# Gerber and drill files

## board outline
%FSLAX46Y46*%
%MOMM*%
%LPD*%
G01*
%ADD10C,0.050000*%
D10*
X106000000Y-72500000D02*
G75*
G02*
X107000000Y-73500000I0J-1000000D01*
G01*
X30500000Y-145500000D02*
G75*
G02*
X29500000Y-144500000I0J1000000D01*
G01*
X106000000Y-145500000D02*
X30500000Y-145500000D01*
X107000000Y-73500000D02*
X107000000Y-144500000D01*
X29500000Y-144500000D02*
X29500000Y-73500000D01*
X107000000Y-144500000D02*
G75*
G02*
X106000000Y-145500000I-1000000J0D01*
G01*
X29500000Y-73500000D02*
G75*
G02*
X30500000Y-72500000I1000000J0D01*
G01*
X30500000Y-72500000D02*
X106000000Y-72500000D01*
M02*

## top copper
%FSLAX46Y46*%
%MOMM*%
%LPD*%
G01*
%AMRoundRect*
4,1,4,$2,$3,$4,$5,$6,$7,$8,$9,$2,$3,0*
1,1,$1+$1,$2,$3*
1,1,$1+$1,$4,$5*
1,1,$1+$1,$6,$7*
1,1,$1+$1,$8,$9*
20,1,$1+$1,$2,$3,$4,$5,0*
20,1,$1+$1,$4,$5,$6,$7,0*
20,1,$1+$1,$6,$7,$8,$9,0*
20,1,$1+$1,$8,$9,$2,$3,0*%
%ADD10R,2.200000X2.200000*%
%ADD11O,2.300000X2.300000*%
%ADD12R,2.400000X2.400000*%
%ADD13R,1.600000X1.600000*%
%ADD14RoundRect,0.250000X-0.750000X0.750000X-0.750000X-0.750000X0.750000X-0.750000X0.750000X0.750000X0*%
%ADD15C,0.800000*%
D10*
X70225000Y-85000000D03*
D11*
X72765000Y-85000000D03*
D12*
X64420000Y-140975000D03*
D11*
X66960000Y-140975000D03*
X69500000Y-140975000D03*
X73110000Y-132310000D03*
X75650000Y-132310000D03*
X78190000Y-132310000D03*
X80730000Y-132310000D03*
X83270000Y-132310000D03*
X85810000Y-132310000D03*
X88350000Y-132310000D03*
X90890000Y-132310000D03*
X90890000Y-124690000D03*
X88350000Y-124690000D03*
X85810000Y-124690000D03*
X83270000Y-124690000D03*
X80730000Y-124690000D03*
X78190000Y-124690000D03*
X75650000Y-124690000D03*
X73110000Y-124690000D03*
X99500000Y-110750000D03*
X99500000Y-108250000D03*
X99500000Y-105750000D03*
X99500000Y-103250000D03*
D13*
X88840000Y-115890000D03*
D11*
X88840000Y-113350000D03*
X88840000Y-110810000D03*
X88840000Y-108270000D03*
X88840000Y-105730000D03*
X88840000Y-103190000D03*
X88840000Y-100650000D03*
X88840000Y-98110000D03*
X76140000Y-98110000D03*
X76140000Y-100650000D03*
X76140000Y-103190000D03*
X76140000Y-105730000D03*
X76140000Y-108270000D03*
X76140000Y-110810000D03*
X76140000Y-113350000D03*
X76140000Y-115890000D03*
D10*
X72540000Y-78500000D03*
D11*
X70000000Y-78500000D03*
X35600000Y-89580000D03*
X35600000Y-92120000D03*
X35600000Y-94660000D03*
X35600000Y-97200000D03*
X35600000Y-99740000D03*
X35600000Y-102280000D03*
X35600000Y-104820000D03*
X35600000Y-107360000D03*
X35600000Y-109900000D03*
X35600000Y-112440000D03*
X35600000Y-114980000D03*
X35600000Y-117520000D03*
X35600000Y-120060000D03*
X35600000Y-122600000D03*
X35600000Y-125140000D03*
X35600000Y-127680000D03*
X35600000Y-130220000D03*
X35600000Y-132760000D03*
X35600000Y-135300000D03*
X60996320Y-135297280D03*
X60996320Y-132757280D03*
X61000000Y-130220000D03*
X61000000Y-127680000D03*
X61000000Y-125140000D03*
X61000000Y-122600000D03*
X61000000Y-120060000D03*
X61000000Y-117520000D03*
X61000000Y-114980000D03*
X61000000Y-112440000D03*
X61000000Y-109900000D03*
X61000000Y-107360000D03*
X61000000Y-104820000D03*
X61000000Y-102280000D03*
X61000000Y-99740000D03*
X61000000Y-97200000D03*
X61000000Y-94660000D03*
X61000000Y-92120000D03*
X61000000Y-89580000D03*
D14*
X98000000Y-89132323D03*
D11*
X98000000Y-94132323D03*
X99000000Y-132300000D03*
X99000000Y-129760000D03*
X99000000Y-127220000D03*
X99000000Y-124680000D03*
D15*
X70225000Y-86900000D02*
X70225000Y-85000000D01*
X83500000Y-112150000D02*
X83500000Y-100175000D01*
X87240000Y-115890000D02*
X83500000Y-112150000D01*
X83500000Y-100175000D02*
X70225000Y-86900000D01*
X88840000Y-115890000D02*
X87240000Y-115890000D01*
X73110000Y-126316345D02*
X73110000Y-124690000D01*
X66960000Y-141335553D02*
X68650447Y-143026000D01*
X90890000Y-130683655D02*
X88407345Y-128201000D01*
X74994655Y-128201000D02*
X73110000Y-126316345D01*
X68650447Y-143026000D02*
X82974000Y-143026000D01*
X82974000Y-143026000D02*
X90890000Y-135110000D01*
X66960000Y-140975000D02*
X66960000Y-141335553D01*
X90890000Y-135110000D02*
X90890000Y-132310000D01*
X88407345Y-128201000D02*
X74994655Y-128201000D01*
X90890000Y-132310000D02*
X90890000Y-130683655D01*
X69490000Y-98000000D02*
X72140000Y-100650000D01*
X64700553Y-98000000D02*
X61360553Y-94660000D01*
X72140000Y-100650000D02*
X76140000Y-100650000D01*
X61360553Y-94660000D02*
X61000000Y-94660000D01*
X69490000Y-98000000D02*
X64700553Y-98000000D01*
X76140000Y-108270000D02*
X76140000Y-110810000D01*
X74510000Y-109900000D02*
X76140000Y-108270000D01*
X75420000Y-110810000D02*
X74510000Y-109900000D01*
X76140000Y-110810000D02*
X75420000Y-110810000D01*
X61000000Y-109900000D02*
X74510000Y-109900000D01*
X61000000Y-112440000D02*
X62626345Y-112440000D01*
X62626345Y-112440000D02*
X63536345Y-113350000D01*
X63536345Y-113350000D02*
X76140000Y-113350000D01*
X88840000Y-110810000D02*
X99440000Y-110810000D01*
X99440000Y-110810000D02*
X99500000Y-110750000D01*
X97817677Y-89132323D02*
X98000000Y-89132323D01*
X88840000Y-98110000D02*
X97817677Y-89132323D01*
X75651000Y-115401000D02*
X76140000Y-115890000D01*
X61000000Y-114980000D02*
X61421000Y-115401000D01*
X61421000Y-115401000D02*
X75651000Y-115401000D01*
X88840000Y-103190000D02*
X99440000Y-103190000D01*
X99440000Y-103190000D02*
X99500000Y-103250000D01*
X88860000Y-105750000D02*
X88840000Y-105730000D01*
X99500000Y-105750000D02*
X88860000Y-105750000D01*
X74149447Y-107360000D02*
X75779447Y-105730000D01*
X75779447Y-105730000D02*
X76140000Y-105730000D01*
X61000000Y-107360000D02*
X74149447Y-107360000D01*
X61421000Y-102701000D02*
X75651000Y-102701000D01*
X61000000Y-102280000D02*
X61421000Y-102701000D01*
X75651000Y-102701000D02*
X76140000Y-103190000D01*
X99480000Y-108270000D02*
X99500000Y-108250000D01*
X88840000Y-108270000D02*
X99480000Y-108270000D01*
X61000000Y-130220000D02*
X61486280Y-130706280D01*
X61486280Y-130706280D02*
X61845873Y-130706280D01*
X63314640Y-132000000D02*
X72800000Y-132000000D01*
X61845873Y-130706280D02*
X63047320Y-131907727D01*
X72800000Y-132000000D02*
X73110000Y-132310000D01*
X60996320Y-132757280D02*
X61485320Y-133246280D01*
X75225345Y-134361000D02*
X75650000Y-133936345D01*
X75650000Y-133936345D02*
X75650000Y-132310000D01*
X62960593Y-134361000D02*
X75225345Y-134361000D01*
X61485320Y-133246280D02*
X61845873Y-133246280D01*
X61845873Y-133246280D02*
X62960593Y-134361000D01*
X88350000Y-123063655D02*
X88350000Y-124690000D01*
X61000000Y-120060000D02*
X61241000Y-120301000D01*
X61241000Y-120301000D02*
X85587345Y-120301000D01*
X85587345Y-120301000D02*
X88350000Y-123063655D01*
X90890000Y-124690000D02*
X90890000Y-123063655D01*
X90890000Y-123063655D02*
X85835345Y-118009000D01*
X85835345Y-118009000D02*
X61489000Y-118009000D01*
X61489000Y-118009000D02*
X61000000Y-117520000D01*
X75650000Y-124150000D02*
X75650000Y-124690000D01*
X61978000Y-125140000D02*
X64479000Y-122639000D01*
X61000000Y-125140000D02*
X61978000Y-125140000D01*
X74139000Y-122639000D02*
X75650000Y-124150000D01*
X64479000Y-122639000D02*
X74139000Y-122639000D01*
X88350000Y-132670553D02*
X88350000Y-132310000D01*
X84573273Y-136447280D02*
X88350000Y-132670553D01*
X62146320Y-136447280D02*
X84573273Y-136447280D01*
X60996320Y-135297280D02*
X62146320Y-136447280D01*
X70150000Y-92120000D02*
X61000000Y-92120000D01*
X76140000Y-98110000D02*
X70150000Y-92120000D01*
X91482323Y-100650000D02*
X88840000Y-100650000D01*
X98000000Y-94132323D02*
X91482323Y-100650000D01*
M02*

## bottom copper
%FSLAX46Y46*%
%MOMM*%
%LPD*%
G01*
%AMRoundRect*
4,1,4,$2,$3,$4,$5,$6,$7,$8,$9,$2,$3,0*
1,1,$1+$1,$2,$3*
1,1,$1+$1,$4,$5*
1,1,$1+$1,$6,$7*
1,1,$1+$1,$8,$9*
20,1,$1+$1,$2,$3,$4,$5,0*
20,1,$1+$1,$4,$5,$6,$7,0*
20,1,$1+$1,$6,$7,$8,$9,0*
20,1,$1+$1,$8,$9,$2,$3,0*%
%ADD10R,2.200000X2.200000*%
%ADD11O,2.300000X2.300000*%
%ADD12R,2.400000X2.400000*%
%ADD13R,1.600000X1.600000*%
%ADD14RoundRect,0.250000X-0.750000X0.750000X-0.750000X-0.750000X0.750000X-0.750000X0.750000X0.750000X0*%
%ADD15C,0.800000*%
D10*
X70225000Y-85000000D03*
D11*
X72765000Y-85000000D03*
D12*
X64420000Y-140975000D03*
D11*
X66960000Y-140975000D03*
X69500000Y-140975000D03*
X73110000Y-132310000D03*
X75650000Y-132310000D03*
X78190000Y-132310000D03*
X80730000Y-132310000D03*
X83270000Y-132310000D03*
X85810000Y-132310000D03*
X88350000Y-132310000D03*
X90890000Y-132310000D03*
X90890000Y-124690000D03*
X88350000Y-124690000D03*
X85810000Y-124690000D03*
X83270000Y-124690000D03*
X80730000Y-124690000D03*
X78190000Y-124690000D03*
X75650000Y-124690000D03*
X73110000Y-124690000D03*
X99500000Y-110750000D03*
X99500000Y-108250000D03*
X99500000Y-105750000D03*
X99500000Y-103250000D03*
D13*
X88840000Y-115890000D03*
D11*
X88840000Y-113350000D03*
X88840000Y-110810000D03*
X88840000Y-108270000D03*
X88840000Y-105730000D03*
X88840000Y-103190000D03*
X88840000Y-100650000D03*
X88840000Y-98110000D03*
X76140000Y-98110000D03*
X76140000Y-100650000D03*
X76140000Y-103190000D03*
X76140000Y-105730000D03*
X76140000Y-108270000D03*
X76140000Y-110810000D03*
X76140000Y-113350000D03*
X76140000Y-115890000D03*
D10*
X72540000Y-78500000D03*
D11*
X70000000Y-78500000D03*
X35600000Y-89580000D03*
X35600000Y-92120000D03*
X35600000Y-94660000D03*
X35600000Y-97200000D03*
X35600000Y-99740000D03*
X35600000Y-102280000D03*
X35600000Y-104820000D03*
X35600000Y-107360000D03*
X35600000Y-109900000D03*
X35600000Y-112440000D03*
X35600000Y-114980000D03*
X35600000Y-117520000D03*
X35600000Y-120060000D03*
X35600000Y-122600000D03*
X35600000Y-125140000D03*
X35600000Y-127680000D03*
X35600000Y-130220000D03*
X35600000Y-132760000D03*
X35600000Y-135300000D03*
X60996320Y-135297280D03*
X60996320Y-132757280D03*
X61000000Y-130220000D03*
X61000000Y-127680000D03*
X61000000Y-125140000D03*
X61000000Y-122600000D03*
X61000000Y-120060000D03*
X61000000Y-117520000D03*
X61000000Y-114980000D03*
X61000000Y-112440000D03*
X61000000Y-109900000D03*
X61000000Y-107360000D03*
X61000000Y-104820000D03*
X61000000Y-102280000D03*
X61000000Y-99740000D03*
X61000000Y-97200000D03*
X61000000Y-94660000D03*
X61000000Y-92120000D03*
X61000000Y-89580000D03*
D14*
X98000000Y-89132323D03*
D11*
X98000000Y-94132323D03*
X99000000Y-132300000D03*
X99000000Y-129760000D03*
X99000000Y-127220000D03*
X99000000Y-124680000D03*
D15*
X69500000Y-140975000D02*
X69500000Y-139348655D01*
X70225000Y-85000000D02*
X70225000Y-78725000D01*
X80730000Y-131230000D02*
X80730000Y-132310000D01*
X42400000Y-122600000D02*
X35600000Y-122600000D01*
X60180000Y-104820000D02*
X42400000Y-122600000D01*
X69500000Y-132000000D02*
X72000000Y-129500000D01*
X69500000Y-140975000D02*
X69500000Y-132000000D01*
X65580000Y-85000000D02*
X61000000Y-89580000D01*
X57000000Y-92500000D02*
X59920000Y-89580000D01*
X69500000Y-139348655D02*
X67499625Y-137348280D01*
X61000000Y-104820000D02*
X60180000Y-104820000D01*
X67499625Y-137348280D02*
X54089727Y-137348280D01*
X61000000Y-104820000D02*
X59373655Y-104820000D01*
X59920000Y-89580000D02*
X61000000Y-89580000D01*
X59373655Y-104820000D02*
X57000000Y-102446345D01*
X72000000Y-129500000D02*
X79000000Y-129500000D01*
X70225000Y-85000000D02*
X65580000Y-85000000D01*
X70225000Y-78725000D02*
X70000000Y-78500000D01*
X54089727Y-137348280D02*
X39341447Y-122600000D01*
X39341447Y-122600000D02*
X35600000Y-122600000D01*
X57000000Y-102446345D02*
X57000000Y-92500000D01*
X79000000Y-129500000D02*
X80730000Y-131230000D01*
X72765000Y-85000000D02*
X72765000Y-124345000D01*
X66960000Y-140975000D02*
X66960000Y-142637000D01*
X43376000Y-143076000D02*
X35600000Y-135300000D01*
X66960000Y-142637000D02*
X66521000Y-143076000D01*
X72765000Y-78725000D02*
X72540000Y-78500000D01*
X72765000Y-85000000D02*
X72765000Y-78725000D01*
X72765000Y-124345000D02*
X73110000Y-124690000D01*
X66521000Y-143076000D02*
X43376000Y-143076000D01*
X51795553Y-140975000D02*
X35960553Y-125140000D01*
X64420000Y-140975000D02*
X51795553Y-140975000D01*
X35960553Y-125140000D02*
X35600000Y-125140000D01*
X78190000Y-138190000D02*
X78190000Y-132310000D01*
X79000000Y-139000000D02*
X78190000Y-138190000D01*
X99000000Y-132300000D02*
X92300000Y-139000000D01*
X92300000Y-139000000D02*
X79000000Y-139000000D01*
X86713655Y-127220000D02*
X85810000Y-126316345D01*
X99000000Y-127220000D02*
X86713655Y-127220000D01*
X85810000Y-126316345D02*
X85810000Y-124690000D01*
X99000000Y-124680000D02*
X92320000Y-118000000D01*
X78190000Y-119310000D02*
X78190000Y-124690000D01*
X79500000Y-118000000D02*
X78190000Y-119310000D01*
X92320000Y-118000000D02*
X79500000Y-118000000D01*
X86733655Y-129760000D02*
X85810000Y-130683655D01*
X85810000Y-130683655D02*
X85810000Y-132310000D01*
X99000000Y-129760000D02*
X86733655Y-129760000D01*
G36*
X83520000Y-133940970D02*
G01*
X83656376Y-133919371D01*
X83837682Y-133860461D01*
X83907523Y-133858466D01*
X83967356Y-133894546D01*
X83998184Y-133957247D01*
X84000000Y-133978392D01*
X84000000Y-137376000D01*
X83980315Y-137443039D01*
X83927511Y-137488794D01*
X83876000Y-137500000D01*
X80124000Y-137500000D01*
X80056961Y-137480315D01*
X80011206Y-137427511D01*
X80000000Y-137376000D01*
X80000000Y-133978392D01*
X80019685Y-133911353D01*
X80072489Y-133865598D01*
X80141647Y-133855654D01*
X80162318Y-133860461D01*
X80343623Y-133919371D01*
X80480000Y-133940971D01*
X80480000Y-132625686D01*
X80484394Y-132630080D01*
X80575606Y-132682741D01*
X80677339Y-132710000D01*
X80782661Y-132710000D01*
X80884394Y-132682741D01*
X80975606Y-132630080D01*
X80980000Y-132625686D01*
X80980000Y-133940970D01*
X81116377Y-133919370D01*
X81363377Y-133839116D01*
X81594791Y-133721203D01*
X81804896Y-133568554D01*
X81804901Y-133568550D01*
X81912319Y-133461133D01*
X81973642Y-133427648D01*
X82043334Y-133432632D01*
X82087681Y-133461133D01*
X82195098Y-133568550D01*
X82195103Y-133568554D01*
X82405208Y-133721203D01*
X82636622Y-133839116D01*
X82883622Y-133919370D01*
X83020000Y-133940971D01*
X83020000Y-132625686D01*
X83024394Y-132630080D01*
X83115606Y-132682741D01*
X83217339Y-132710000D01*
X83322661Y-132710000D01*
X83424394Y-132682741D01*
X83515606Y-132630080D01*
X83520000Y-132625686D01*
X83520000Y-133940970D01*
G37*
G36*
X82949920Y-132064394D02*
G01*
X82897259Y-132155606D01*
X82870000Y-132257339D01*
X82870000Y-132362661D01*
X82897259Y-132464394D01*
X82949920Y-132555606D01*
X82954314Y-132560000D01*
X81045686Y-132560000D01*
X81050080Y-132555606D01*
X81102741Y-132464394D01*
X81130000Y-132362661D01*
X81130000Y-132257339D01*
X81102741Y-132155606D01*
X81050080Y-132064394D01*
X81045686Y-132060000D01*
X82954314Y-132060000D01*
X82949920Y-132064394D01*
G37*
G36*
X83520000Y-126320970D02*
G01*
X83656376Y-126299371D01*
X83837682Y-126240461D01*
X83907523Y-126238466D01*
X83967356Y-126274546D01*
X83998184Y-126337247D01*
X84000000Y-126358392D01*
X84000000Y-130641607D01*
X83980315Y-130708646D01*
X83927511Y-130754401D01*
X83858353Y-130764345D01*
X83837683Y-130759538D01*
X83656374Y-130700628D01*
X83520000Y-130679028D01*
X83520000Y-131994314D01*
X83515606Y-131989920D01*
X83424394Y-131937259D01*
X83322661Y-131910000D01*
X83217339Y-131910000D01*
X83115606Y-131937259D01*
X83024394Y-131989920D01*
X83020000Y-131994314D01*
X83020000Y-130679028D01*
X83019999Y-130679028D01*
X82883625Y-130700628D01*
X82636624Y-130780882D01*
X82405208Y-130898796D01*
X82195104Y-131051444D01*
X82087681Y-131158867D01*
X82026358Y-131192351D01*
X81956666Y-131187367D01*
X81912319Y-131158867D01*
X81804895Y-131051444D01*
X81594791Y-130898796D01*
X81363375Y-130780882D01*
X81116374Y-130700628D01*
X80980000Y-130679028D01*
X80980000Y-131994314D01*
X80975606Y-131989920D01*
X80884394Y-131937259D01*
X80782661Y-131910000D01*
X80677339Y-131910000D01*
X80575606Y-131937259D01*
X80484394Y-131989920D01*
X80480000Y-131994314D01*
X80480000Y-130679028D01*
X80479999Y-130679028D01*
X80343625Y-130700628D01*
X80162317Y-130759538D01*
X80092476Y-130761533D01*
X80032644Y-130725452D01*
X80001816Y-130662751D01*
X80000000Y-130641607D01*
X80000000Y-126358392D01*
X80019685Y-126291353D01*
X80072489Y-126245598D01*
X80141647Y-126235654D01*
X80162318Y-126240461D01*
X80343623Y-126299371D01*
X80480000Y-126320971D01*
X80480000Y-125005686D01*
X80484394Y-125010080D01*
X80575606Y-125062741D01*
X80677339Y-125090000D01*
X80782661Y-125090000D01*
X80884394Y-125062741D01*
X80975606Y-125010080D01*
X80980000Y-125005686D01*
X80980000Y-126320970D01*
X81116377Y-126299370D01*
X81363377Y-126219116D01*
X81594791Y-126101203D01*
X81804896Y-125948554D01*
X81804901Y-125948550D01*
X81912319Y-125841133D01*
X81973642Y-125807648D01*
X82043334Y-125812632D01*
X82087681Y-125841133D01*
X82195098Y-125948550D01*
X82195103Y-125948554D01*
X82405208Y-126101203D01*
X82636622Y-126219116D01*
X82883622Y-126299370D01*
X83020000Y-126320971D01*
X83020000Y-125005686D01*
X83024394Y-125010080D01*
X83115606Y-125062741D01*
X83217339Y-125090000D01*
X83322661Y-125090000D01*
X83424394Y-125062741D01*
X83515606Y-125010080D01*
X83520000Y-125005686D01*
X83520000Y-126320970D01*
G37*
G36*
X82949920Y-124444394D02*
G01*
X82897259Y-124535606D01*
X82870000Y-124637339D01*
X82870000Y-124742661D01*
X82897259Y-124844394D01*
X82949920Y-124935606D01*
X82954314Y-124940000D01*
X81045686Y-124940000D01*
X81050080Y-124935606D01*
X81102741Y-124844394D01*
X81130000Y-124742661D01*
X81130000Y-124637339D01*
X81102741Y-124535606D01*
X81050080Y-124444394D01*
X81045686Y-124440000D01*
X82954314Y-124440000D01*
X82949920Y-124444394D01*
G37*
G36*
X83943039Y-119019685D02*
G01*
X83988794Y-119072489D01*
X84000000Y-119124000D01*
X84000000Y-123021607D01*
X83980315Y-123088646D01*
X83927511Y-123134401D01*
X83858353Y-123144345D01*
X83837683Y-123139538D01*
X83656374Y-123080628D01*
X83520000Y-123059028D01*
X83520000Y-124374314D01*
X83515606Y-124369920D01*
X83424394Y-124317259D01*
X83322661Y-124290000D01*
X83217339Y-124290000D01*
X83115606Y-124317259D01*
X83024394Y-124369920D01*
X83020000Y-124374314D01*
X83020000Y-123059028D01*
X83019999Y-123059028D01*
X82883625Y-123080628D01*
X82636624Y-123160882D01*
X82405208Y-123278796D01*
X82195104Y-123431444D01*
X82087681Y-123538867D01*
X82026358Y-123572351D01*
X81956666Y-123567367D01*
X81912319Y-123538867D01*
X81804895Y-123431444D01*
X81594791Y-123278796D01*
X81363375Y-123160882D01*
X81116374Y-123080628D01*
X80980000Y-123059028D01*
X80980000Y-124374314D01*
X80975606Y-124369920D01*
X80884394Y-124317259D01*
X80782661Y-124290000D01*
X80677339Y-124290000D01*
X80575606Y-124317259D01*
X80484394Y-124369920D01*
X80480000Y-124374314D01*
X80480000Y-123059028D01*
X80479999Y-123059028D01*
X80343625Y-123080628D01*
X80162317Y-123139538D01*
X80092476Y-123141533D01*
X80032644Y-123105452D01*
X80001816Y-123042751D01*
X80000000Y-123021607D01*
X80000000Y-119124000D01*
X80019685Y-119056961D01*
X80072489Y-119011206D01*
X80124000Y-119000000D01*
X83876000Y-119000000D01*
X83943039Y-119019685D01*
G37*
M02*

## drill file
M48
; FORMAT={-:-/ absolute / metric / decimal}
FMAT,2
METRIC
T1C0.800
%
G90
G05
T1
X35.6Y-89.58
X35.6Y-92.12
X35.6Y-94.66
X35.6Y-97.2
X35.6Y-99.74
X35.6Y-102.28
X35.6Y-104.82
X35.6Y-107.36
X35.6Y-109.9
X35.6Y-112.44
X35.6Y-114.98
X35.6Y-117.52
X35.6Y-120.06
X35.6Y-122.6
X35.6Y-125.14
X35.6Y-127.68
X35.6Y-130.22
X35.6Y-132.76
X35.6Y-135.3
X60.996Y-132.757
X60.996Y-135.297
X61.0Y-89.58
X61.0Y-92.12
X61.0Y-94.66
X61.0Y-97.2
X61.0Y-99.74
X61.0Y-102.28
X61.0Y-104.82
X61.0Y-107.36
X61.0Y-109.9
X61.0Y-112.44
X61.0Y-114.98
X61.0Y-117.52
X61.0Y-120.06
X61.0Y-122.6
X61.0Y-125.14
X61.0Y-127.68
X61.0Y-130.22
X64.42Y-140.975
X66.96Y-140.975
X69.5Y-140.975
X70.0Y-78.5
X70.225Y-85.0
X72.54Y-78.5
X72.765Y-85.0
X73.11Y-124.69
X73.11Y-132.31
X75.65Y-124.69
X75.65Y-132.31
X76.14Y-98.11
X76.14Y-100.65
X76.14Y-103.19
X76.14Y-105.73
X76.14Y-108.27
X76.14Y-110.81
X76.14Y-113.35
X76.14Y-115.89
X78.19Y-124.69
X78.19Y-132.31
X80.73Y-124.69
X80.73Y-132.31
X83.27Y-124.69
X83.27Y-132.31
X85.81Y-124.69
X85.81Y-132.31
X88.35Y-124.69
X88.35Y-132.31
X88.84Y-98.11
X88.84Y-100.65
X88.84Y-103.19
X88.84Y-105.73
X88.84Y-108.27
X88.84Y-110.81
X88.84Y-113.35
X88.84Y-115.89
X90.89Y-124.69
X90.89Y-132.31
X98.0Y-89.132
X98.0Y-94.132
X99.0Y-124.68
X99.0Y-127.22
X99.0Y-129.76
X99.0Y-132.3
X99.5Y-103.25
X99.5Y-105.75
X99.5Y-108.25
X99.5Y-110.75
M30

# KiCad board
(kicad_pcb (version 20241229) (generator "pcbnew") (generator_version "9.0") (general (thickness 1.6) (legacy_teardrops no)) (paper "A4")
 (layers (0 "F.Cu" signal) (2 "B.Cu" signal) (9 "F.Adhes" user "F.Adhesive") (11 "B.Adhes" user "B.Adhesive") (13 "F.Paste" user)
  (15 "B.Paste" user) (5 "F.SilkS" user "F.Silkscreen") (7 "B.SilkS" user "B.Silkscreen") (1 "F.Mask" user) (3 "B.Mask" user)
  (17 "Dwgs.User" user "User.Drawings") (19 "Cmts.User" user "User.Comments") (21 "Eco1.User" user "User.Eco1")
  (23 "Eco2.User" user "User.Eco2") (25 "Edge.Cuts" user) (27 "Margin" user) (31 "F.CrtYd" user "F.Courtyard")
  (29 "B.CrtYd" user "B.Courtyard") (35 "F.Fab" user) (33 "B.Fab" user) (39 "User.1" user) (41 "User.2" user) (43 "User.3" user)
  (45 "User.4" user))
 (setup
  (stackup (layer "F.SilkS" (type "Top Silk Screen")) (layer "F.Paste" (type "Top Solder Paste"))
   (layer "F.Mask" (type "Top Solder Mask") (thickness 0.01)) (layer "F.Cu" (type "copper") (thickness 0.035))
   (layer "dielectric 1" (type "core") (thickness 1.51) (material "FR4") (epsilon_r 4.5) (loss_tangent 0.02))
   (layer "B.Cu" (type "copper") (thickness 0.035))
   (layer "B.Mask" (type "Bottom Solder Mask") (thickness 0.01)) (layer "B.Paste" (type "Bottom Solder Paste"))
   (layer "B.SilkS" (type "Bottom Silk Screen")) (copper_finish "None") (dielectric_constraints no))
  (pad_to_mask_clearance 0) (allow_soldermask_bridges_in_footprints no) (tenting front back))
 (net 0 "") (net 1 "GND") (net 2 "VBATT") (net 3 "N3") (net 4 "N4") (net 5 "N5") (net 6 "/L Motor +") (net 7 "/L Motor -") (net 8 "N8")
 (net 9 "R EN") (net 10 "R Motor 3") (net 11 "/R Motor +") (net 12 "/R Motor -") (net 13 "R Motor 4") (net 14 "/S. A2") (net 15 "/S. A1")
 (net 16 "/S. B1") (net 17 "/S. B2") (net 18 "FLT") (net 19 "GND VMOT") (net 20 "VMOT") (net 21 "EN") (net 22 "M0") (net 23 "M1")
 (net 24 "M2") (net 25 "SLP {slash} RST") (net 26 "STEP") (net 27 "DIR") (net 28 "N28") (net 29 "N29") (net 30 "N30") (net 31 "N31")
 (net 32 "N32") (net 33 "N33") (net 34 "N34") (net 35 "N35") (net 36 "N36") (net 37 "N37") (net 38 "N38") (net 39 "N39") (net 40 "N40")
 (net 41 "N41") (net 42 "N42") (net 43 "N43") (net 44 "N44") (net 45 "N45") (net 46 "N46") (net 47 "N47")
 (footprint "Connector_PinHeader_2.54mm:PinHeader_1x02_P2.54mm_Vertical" (layer "F.Cu") (at 70.225 85 90)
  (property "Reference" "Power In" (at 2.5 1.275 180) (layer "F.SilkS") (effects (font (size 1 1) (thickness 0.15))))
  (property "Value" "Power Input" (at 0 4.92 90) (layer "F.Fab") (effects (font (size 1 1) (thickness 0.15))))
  (pad "1" thru_hole rect (at 0 0 90) (size 2.2 2.2) (drill 0.8) (layers "*.Cu" "*.Mask") (remove_unused_layers no) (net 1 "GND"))
  (pad "2" thru_hole oval (at 0 2.54 90) (size 2.3 2.3) (drill 0.8) (layers "*.Cu" "*.Mask") (remove_unused_layers no) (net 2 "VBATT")))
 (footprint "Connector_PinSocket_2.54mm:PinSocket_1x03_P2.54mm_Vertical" (layer "F.Cu") (at 64.42 140.975 90)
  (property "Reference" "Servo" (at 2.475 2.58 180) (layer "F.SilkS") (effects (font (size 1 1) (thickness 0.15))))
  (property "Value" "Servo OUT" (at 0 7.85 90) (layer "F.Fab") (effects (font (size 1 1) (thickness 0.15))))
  (pad "1" thru_hole rect (at 0 0 90) (size 2.4 2.4) (drill 0.8) (layers "*.Cu" "*.Mask") (remove_unused_layers no) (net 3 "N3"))
  (pad "2" thru_hole oval (at 0 2.54 90) (size 2.3 2.3) (drill 0.8) (layers "*.Cu" "*.Mask") (remove_unused_layers no) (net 2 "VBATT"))
  (pad "3" thru_hole oval (at 0 5.08 90) (size 2.3 2.3) (drill 0.8) (layers "*.Cu" "*.Mask") (remove_unused_layers no) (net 1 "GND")))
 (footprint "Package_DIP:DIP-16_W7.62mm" (layer "F.Cu") (at 73.11 132.31 90)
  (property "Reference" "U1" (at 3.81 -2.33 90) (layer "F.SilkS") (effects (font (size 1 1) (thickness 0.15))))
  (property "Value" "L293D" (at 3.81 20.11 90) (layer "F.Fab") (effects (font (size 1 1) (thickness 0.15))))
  (pad "1" thru_hole oval (at 0 0 90) (size 2.3 2.3) (drill 0.8) (layers "*.Cu" "*.Mask") (remove_unused_layers no) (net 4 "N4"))
  (pad "2" thru_hole oval (at 0 2.54 90) (size 2.3 2.3) (drill 0.8) (layers "*.Cu" "*.Mask") (remove_unused_layers no) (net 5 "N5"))
  (pad "3" thru_hole oval (at 0 5.08 90) (size 2.3 2.3) (drill 0.8) (layers "*.Cu" "*.Mask") (remove_unused_layers no) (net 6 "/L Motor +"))
  (pad "4" thru_hole oval (at 0 7.62 90) (size 2.3 2.3) (drill 0.8) (layers "*.Cu" "*.Mask") (remove_unused_layers no) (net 1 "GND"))
  (pad "5" thru_hole oval (at 0 10.16 90) (size 2.3 2.3) (drill 0.8) (layers "*.Cu" "*.Mask") (remove_unused_layers no) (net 1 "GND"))
  (pad "6" thru_hole oval (at 0 12.7 90) (size 2.3 2.3) (drill 0.8) (layers "*.Cu" "*.Mask") (remove_unused_layers no) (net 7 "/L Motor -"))
  (pad "7" thru_hole oval (at 0 15.24 90) (size 2.3 2.3) (drill 0.8) (layers "*.Cu" "*.Mask") (remove_unused_layers no) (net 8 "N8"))
  (pad "8" thru_hole oval (at 0 17.78 90) (size 2.3 2.3) (drill 0.8) (layers "*.Cu" "*.Mask") (remove_unused_layers no) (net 2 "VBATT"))
  (pad "9" thru_hole oval (at 7.62 17.78 90) (size 2.3 2.3) (drill 0.8) (layers "*.Cu" "*.Mask") (remove_unused_layers no) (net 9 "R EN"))
  (pad "10" thru_hole oval (at 7.62 15.24 90) (size 2.3 2.3) (drill 0.8) (layers "*.Cu" "*.Mask") (remove_unused_layers no)
   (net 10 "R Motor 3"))
  (pad "11" thru_hole oval (at 7.62 12.7 90) (size 2.3 2.3) (drill 0.8) (layers "*.Cu" "*.Mask") (remove_unused_layers no)
   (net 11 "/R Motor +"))
  (pad "12" thru_hole oval (at 7.62 10.16 90) (size 2.3 2.3) (drill 0.8) (layers "*.Cu" "*.Mask") (remove_unused_layers no) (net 1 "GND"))
  (pad "13" thru_hole oval (at 7.62 7.62 90) (size 2.3 2.3) (drill 0.8) (layers "*.Cu" "*.Mask") (remove_unused_layers no) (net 1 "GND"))
  (pad "14" thru_hole oval (at 7.62 5.08 90) (size 2.3 2.3) (drill 0.8) (layers "*.Cu" "*.Mask") (remove_unused_layers no)
   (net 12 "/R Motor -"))
  (pad "15" thru_hole oval (at 7.62 2.54 90) (size 2.3 2.3) (drill 0.8) (layers "*.Cu" "*.Mask") (remove_unused_layers no)
   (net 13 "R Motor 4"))
  (pad "16" thru_hole oval (at 7.62 0 90) (size 2.3 2.3) (drill 0.8) (layers "*.Cu" "*.Mask") (remove_unused_layers no) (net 2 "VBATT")))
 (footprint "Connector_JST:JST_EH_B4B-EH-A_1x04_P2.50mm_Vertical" (layer "F.Cu") (at 99.5 110.75 90)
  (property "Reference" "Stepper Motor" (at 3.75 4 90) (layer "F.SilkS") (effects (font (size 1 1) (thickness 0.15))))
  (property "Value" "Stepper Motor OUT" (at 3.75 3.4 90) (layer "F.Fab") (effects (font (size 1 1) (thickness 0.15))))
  (pad "1" thru_hole oval (at 0 0 90) (size 2.3 2.3) (drill 0.8) (layers "*.Cu" "*.Mask") (remove_unused_layers no) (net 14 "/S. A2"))
  (pad "2" thru_hole oval (at 2.5 0 90) (size 2.3 2.3) (drill 0.8) (layers "*.Cu" "*.Mask") (remove_unused_layers no) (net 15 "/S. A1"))
  (pad "3" thru_hole oval (at 5 0 90) (size 2.3 2.3) (drill 0.8) (layers "*.Cu" "*.Mask") (remove_unused_layers no) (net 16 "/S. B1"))
  (pad "4" thru_hole oval (at 7.5 0 90) (size 2.3 2.3) (drill 0.8) (layers "*.Cu" "*.Mask") (remove_unused_layers no) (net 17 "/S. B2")))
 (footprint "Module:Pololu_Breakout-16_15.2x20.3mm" (layer "F.Cu") (at 88.84 115.89 180)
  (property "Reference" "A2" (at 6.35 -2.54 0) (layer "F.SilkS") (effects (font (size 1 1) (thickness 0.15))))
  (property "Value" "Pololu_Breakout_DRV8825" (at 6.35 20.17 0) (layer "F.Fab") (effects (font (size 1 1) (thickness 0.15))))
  (pad "1" thru_hole rect (at 0 0 180) (size 1.6 1.6) (drill 0.8) (layers "*.Cu" "*.Mask") (remove_unused_layers no) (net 1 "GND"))
  (pad "2" thru_hole oval (at 0 2.54 180) (size 2.3 2.3) (drill 0.8) (layers "*.Cu" "*.Mask") (remove_unused_layers no) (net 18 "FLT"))
  (pad "3" thru_hole oval (at 0 5.08 180) (size 2.3 2.3) (drill 0.8) (layers "*.Cu" "*.Mask") (remove_unused_layers no) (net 14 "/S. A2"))
  (pad "4" thru_hole oval (at 0 7.62 180) (size 2.3 2.3) (drill 0.8) (layers "*.Cu" "*.Mask") (remove_unused_layers no) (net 15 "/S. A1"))
  (pad "5" thru_hole oval (at 0 10.16 180) (size 2.3 2.3) (drill 0.8) (layers "*.Cu" "*.Mask") (remove_unused_layers no) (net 16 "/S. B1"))
  (pad "6" thru_hole oval (at 0 12.7 180) (size 2.3 2.3) (drill 0.8) (layers "*.Cu" "*.Mask") (remove_unused_layers no) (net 17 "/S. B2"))
  (pad "7" thru_hole oval (at 0 15.24 180) (size 2.3 2.3) (drill 0.8) (layers "*.Cu" "*.Mask") (remove_unused_layers no) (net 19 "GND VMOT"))
  (pad "8" thru_hole oval (at 0 17.78 180) (size 2.3 2.3) (drill 0.8) (layers "*.Cu" "*.Mask") (remove_unused_layers no) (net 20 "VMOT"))
  (pad "9" thru_hole oval (at 12.7 17.78 180) (size 2.3 2.3) (drill 0.8) (layers "*.Cu" "*.Mask") (remove_unused_layers no) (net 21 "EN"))
  (pad "10" thru_hole oval (at 12.7 15.24 180) (size 2.3 2.3) (drill 0.8) (layers "*.Cu" "*.Mask") (remove_unused_layers no) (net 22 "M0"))
  (pad "11" thru_hole oval (at 12.7 12.7 180) (size 2.3 2.3) (drill 0.8) (layers "*.Cu" "*.Mask") (remove_unused_layers no) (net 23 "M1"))
  (pad "12" thru_hole oval (at 12.7 10.16 180) (size 2.3 2.3) (drill 0.8) (layers "*.Cu" "*.Mask") (remove_unused_layers no) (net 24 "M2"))
  (pad "13" thru_hole oval (at 12.7 7.62 180) (size 2.3 2.3) (drill 0.8) (layers "*.Cu" "*.Mask") (remove_unused_layers no)
   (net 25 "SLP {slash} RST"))
  (pad "14" thru_hole oval (at 12.7 5.08 180) (size 2.3 2.3) (drill 0.8) (layers "*.Cu" "*.Mask") (remove_unused_layers no)
   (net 25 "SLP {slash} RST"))
  (pad "15" thru_hole oval (at 12.7 2.54 180) (size 2.3 2.3) (drill 0.8) (layers "*.Cu" "*.Mask") (remove_unused_layers no) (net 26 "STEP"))
  (pad "16" thru_hole oval (at 12.7 0 180) (size 2.3 2.3) (drill 0.8) (layers "*.Cu" "*.Mask") (remove_unused_layers no) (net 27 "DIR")))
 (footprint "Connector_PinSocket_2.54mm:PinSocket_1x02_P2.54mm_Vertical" (layer "F.Cu") (at 72.54 78.5 -90)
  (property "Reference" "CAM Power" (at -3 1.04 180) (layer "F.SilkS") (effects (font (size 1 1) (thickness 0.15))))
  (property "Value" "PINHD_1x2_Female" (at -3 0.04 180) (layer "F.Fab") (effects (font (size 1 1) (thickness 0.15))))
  (pad "1" thru_hole rect (at 0 0 270) (size 2.2 2.2) (drill 0.8) (layers "*.Cu" "*.Mask") (remove_unused_layers no) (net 2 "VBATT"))
  (pad "2" thru_hole oval (at 0 2.54 270) (size 2.3 2.3) (drill 0.8) (layers "*.Cu" "*.Mask") (remove_unused_layers no) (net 1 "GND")))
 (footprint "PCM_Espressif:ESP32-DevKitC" (layer "F.Cu") (at 35.6 89.58)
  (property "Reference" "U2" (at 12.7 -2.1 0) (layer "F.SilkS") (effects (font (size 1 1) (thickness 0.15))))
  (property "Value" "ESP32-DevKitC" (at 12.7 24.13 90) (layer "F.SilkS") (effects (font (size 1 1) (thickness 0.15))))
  (pad "1" thru_hole oval (at 0 0) (size 2.3 2.3) (drill 0.8) (layers "*.Cu" "*.Mask") (remove_unused_layers no) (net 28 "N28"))
  (pad "2" thru_hole oval (at 0 2.54) (size 2.3 2.3) (drill 0.8) (layers "*.Cu" "*.Mask") (remove_unused_layers no) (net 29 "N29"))
  (pad "3" thru_hole oval (at 0 5.08) (size 2.3 2.3) (drill 0.8) (layers "*.Cu" "*.Mask") (remove_unused_layers no) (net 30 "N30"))
  (pad "4" thru_hole oval (at 0 7.62) (size 2.3 2.3) (drill 0.8) (layers "*.Cu" "*.Mask") (remove_unused_layers no) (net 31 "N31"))
  (pad "5" thru_hole oval (at 0 10.16) (size 2.3 2.3) (drill 0.8) (layers "*.Cu" "*.Mask") (remove_unused_layers no) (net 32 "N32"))
  (pad "6" thru_hole oval (at 0 12.7) (size 2.3 2.3) (drill 0.8) (layers "*.Cu" "*.Mask") (remove_unused_layers no) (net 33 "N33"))
  (pad "7" thru_hole oval (at 0 15.24) (size 2.3 2.3) (drill 0.8) (layers "*.Cu" "*.Mask") (remove_unused_layers no) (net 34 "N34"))
  (pad "8" thru_hole oval (at 0 17.78) (size 2.3 2.3) (drill 0.8) (layers "*.Cu" "*.Mask") (remove_unused_layers no) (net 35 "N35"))
  (pad "9" thru_hole oval (at 0 20.32) (size 2.3 2.3) (drill 0.8) (layers "*.Cu" "*.Mask") (remove_unused_layers no) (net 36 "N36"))
  (pad "10" thru_hole oval (at 0 22.86) (size 2.3 2.3) (drill 0.8) (layers "*.Cu" "*.Mask") (remove_unused_layers no) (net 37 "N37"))
  (pad "11" thru_hole oval (at 0 25.4) (size 2.3 2.3) (drill 0.8) (layers "*.Cu" "*.Mask") (remove_unused_layers no) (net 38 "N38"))
  (pad "12" thru_hole oval (at 0 27.94) (size 2.3 2.3) (drill 0.8) (layers "*.Cu" "*.Mask") (remove_unused_layers no) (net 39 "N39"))
  (pad "13" thru_hole oval (at 0 30.48) (size 2.3 2.3) (drill 0.8) (layers "*.Cu" "*.Mask") (remove_unused_layers no) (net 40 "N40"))
  (pad "14" thru_hole oval (at 0 33.02) (size 2.3 2.3) (drill 0.8) (layers "*.Cu" "*.Mask") (remove_unused_layers no) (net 1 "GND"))
  (pad "15" thru_hole oval (at 0 35.56) (size 2.3 2.3) (drill 0.8) (layers "*.Cu" "*.Mask") (remove_unused_layers no) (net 3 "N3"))
  (pad "16" thru_hole oval (at 0 38.1) (size 2.3 2.3) (drill 0.8) (layers "*.Cu" "*.Mask") (remove_unused_layers no) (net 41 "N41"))
  (pad "17" thru_hole oval (at 0 40.64) (size 2.3 2.3) (drill 0.8) (layers "*.Cu" "*.Mask") (remove_unused_layers no) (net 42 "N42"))
  (pad "18" thru_hole oval (at 0 43.18) (size 2.3 2.3) (drill 0.8) (layers "*.Cu" "*.Mask") (remove_unused_layers no) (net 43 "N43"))
  (pad "19" thru_hole oval (at 0 45.72) (size 2.3 2.3) (drill 0.8) (layers "*.Cu" "*.Mask") (remove_unused_layers no) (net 2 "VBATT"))
  (pad "20" thru_hole oval (at 25.39632 45.71728) (size 2.3 2.3) (drill 0.8) (layers "*.Cu" "*.Mask") (remove_unused_layers no) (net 8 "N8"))
  (pad "21" thru_hole oval (at 25.39632 43.17728) (size 2.3 2.3) (drill 0.8) (layers "*.Cu" "*.Mask") (remove_unused_layers no) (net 5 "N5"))
  (pad "22" thru_hole oval (at 25.4 40.64) (size 2.3 2.3) (drill 0.8) (layers "*.Cu" "*.Mask") (remove_unused_layers no) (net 4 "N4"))
  (pad "23" thru_hole oval (at 25.4 38.1) (size 2.3 2.3) (drill 0.8) (layers "*.Cu" "*.Mask") (remove_unused_layers no) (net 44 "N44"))
  (pad "24" thru_hole oval (at 25.4 35.56) (size 2.3 2.3) (drill 0.8) (layers "*.Cu" "*.Mask") (remove_unused_layers no)
   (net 13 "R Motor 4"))
  (pad "25" thru_hole oval (at 25.4 33.02) (size 2.3 2.3) (drill 0.8) (layers "*.Cu" "*.Mask") (remove_unused_layers no) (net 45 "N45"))
  (pad "26" thru_hole oval (at 25.4 30.48) (size 2.3 2.3) (drill 0.8) (layers "*.Cu" "*.Mask") (remove_unused_layers no)
   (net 10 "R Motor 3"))
  (pad "27" thru_hole oval (at 25.4 27.94) (size 2.3 2.3) (drill 0.8) (layers "*.Cu" "*.Mask") (remove_unused_layers no) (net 9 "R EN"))
  (pad "28" thru_hole oval (at 25.4 25.4) (size 2.3 2.3) (drill 0.8) (layers "*.Cu" "*.Mask") (remove_unused_layers no) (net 27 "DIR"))
  (pad "29" thru_hole oval (at 25.4 22.86) (size 2.3 2.3) (drill 0.8) (layers "*.Cu" "*.Mask") (remove_unused_layers no) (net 26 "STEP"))
  (pad "30" thru_hole oval (at 25.4 20.32) (size 2.3 2.3) (drill 0.8) (layers "*.Cu" "*.Mask") (remove_unused_layers no)
   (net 25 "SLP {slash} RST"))
  (pad "31" thru_hole oval (at 25.4 17.78) (size 2.3 2.3) (drill 0.8) (layers "*.Cu" "*.Mask") (remove_unused_layers no) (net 24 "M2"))
  (pad "32" thru_hole oval (at 25.4 15.24) (size 2.3 2.3) (drill 0.8) (layers "*.Cu" "*.Mask") (remove_unused_layers no) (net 1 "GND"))
  (pad "33" thru_hole oval (at 25.4 12.7) (size 2.3 2.3) (drill 0.8) (layers "*.Cu" "*.Mask") (remove_unused_layers no) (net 23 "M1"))
  (pad "34" thru_hole oval (at 25.4 10.16) (size 2.3 2.3) (drill 0.8) (layers "*.Cu" "*.Mask") (remove_unused_layers no) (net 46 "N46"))
  (pad "35" thru_hole oval (at 25.4 7.62) (size 2.3 2.3) (drill 0.8) (layers "*.Cu" "*.Mask") (remove_unused_layers no) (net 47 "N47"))
  (pad "36" thru_hole oval (at 25.4 5.08) (size 2.3 2.3) (drill 0.8) (layers "*.Cu" "*.Mask") (remove_unused_layers no) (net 22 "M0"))
  (pad "37" thru_hole oval (at 25.4 2.54) (size 2.3 2.3) (drill 0.8) (layers "*.Cu" "*.Mask") (remove_unused_layers no) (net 21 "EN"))
  (pad "38" thru_hole oval (at 25.4 0) (size 2.3 2.3) (drill 0.8) (layers "*.Cu" "*.Mask") (remove_unused_layers no) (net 1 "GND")))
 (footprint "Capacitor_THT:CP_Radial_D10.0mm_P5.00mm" (layer "F.Cu") (at 98 89.132323 -90)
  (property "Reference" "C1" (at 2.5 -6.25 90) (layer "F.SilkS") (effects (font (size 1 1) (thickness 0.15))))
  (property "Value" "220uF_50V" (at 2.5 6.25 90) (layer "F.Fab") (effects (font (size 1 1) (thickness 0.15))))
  (pad "1" thru_hole roundrect (at 0 0 270) (size 2 2) (drill 0.8) (layers "*.Cu" "*.Mask") (remove_unused_layers no)
   (roundrect_rratio 0.125) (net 20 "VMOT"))
  (pad "2" thru_hole oval (at 5 0 270) (size 2.3 2.3) (drill 0.8) (layers "*.Cu" "*.Mask") (remove_unused_layers no) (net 19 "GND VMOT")))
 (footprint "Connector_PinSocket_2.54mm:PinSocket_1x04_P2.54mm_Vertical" (layer "F.Cu") (at 99 132.3 180)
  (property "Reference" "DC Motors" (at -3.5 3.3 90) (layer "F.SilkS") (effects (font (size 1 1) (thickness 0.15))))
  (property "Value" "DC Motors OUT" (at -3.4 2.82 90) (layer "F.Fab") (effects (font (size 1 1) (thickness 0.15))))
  (pad "1" thru_hole oval (at 0 0 180) (size 2.3 2.3) (drill 0.8) (layers "*.Cu" "*.Mask") (remove_unused_layers no) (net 6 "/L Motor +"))
  (pad "2" thru_hole oval (at 0 2.54 180) (size 2.3 2.3) (drill 0.8) (layers "*.Cu" "*.Mask") (remove_unused_layers no) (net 7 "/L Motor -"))
  (pad "3" thru_hole oval (at 0 5.08 180) (size 2.3 2.3) (drill 0.8) (layers "*.Cu" "*.Mask") (remove_unused_layers no)
   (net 11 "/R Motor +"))
  (pad "4" thru_hole oval (at 0 7.62 180) (size 2.3 2.3) (drill 0.8) (layers "*.Cu" "*.Mask") (remove_unused_layers no)
   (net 12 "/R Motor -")))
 (gr_arc (start 106 72.5) (mid 106.707107 72.792893) (end 107 73.5) (stroke (width 0.05) (type default)) (layer "Edge.Cuts"))
 (gr_arc (start 30.5 145.5) (mid 29.792893 145.207107) (end 29.5 144.5) (stroke (width 0.05) (type default)) (layer "Edge.Cuts"))
 (gr_line (start 106 145.5) (end 30.5 145.5) (stroke (width 0.05) (type default)) (layer "Edge.Cuts"))
 (gr_line (start 107 73.5) (end 107 144.5) (stroke (width 0.05) (type default)) (layer "Edge.Cuts"))
 (gr_line (start 29.5 144.5) (end 29.5 73.5) (stroke (width 0.05) (type default)) (layer "Edge.Cuts"))
 (gr_arc (start 107 144.5) (mid 106.707107 145.207107) (end 106 145.5) (stroke (width 0.05) (type default)) (layer "Edge.Cuts"))
 (gr_arc (start 29.5 73.5) (mid 29.792893 72.792893) (end 30.5 72.5) (stroke (width 0.05) (type default)) (layer "Edge.Cuts"))
 (gr_line (start 30.5 72.5) (end 106 72.5) (stroke (width 0.05) (type default)) (layer "Edge.Cuts"))
 (segment (start 70.225 86.9) (end 70.225 85) (width 0.8) (layer "F.Cu") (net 1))
 (segment (start 83.5 112.15) (end 83.5 100.175) (width 0.8) (layer "F.Cu") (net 1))
 (segment (start 87.24 115.89) (end 83.5 112.15) (width 0.8) (layer "F.Cu") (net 1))
 (segment (start 83.5 100.175) (end 70.225 86.9) (width 0.8) (layer "F.Cu") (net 1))
 (segment (start 88.84 115.89) (end 87.24 115.89) (width 0.8) (layer "F.Cu") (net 1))
 (segment (start 69.5 140.975) (end 69.5 139.348655) (width 0.8) (layer "B.Cu") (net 1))
 (segment (start 70.225 85) (end 70.225 78.725) (width 0.8) (layer "B.Cu") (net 1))
 (segment (start 80.73 131.23) (end 80.73 132.31) (width 0.8) (layer "B.Cu") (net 1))
 (segment (start 42.4 122.6) (end 35.6 122.6) (width 0.8) (layer "B.Cu") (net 1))
 (segment (start 60.18 104.82) (end 42.4 122.6) (width 0.8) (layer "B.Cu") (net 1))
 (segment (start 69.5 132) (end 72 129.5) (width 0.8) (layer "B.Cu") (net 1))
 (segment (start 69.5 140.975) (end 69.5 132) (width 0.8) (layer "B.Cu") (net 1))
 (segment (start 65.58 85) (end 61 89.58) (width 0.8) (layer "B.Cu") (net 1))
 (segment (start 57 92.5) (end 59.92 89.58) (width 0.8) (layer "B.Cu") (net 1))
 (segment (start 69.5 139.348655) (end 67.499625 137.34828) (width 0.8) (layer "B.Cu") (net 1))
 (segment (start 61 104.82) (end 60.18 104.82) (width 0.8) (layer "B.Cu") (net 1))
 (segment (start 67.499625 137.34828) (end 54.089727 137.34828) (width 0.8) (layer "B.Cu") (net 1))
 (segment (start 61 104.82) (end 59.373655 104.82) (width 0.8) (layer "B.Cu") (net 1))
 (segment (start 59.92 89.58) (end 61 89.58) (width 0.8) (layer "B.Cu") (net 1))
 (segment (start 59.373655 104.82) (end 57 102.446345) (width 0.8) (layer "B.Cu") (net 1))
 (segment (start 72 129.5) (end 79 129.5) (width 0.8) (layer "B.Cu") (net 1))
 (segment (start 70.225 85) (end 65.58 85) (width 0.8) (layer "B.Cu") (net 1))
 (segment (start 70.225 78.725) (end 70 78.5) (width 0.8) (layer "B.Cu") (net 1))
 (segment (start 54.089727 137.34828) (end 39.341447 122.6) (width 0.8) (layer "B.Cu") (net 1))
 (segment (start 39.341447 122.6) (end 35.6 122.6) (width 0.8) (layer "B.Cu") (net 1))
 (segment (start 57 102.446345) (end 57 92.5) (width 0.8) (layer "B.Cu") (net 1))
 (segment (start 79 129.5) (end 80.73 131.23) (width 0.8) (layer "B.Cu") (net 1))
 (segment (start 73.11 126.316345) (end 73.11 124.69) (width 0.8) (layer "F.Cu") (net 2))
 (segment (start 66.96 141.335553) (end 68.650447 143.026) (width 0.8) (layer "F.Cu") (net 2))
 (segment (start 90.89 130.683655) (end 88.407345 128.201) (width 0.8) (layer "F.Cu") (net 2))
 (segment (start 74.994655 128.201) (end 73.11 126.316345) (width 0.8) (layer "F.Cu") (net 2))
 (segment (start 68.650447 143.026) (end 82.974 143.026) (width 0.8) (layer "F.Cu") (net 2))
 (segment (start 82.974 143.026) (end 90.89 135.11) (width 0.8) (layer "F.Cu") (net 2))
 (segment (start 66.96 140.975) (end 66.96 141.335553) (width 0.8) (layer "F.Cu") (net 2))
 (segment (start 90.89 135.11) (end 90.89 132.31) (width 0.8) (layer "F.Cu") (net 2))
 (segment (start 88.407345 128.201) (end 74.994655 128.201) (width 0.8) (layer "F.Cu") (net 2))
 (segment (start 90.89 132.31) (end 90.89 130.683655) (width 0.8) (layer "F.Cu") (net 2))
 (segment (start 72.765 85) (end 72.765 124.345) (width 0.8) (layer "B.Cu") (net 2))
 (segment (start 66.96 140.975) (end 66.96 142.637) (width 0.8) (layer "B.Cu") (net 2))
 (segment (start 43.376 143.076) (end 35.6 135.3) (width 0.8) (layer "B.Cu") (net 2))
 (segment (start 66.96 142.637) (end 66.521 143.076) (width 0.8) (layer "B.Cu") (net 2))
 (segment (start 72.765 78.725) (end 72.54 78.5) (width 0.8) (layer "B.Cu") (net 2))
 (segment (start 72.765 85) (end 72.765 78.725) (width 0.8) (layer "B.Cu") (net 2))
 (segment (start 72.765 124.345) (end 73.11 124.69) (width 0.8) (layer "B.Cu") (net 2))
 (segment (start 66.521 143.076) (end 43.376 143.076) (width 0.8) (layer "B.Cu") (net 2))
 (segment (start 69.49 98) (end 72.14 100.65) (width 0.8) (layer "F.Cu") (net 22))
 (segment (start 64.700553 98) (end 61.360553 94.66) (width 0.8) (layer "F.Cu") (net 22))
 (segment (start 72.14 100.65) (end 76.14 100.65) (width 0.8) (layer "F.Cu") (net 22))
 (segment (start 61.360553 94.66) (end 61 94.66) (width 0.8) (layer "F.Cu") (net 22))
 (segment (start 69.49 98) (end 64.700553 98) (width 0.8) (layer "F.Cu") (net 22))
 (segment (start 76.14 108.27) (end 76.14 110.81) (width 0.8) (layer "F.Cu") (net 25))
 (segment (start 74.51 109.9) (end 76.14 108.27) (width 0.8) (layer "F.Cu") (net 25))
 (segment (start 75.42 110.81) (end 74.51 109.9) (width 0.8) (layer "F.Cu") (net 25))
 (segment (start 76.14 110.81) (end 75.42 110.81) (width 0.8) (layer "F.Cu") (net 25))
 (segment (start 61 109.9) (end 74.51 109.9) (width 0.8) (layer "F.Cu") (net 25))
 (segment (start 61 112.44) (end 62.626345 112.44) (width 0.8) (layer "F.Cu") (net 26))
 (segment (start 62.626345 112.44) (end 63.536345 113.35) (width 0.8) (layer "F.Cu") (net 26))
 (segment (start 63.536345 113.35) (end 76.14 113.35) (width 0.8) (layer "F.Cu") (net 26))
 (segment (start 88.84 110.81) (end 99.44 110.81) (width 0.8) (layer "F.Cu") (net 14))
 (segment (start 99.44 110.81) (end 99.5 110.75) (width 0.8) (layer "F.Cu") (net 14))
 (segment (start 97.817677 89.132323) (end 98 89.132323) (width 0.8) (layer "F.Cu") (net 20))
 (segment (start 88.84 98.11) (end 97.817677 89.132323) (width 0.8) (layer "F.Cu") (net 20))
 (segment (start 75.651 115.401) (end 76.14 115.89) (width 0.8) (layer "F.Cu") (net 27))
 (segment (start 61 114.98) (end 61.421 115.401) (width 0.8) (layer "F.Cu") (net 27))
 (segment (start 61.421 115.401) (end 75.651 115.401) (width 0.8) (layer "F.Cu") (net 27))
 (segment (start 88.84 103.19) (end 99.44 103.19) (width 0.8) (layer "F.Cu") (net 17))
 (segment (start 99.44 103.19) (end 99.5 103.25) (width 0.8) (layer "F.Cu") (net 17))
 (segment (start 88.86 105.75) (end 88.84 105.73) (width 0.8) (layer "F.Cu") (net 16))
 (segment (start 99.5 105.75) (end 88.86 105.75) (width 0.8) (layer "F.Cu") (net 16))
 (segment (start 74.149447 107.36) (end 75.779447 105.73) (width 0.8) (layer "F.Cu") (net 24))
 (segment (start 75.779447 105.73) (end 76.14 105.73) (width 0.8) (layer "F.Cu") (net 24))
 (segment (start 61 107.36) (end 74.149447 107.36) (width 0.8) (layer "F.Cu") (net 24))
 (segment (start 61.421 102.701) (end 75.651 102.701) (width 0.8) (layer "F.Cu") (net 23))
 (segment (start 61 102.28) (end 61.421 102.701) (width 0.8) (layer "F.Cu") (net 23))
 (segment (start 75.651 102.701) (end 76.14 103.19) (width 0.8) (layer "F.Cu") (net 23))
 (segment (start 51.795553 140.975) (end 35.960553 125.14) (width 0.8) (layer "B.Cu") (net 3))
 (segment (start 64.42 140.975) (end 51.795553 140.975) (width 0.8) (layer "B.Cu") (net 3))
 (segment (start 35.960553 125.14) (end 35.6 125.14) (width 0.8) (layer "B.Cu") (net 3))
 (segment (start 99.48 108.27) (end 99.5 108.25) (width 0.8) (layer "F.Cu") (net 15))
 (segment (start 88.84 108.27) (end 99.48 108.27) (width 0.8) (layer "F.Cu") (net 15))
 (segment (start 78.19 138.19) (end 78.19 132.31) (width 0.8) (layer "B.Cu") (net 6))
 (segment (start 79 139) (end 78.19 138.19) (width 0.8) (layer "B.Cu") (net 6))
 (segment (start 99 132.3) (end 92.3 139) (width 0.8) (layer "B.Cu") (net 6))
 (segment (start 92.3 139) (end 79 139) (width 0.8) (layer "B.Cu") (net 6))
 (segment (start 86.713655 127.22) (end 85.81 126.316345) (width 0.8) (layer "B.Cu") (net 11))
 (segment (start 99 127.22) (end 86.713655 127.22) (width 0.8) (layer "B.Cu") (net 11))
 (segment (start 85.81 126.316345) (end 85.81 124.69) (width 0.8) (layer "B.Cu") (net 11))
 (segment (start 99 124.68) (end 92.32 118) (width 0.8) (layer "B.Cu") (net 12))
 (segment (start 78.19 119.31) (end 78.19 124.69) (width 0.8) (layer "B.Cu") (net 12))
 (segment (start 79.5 118) (end 78.19 119.31) (width 0.8) (layer "B.Cu") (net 12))
 (segment (start 92.32 118) (end 79.5 118) (width 0.8) (layer "B.Cu") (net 12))
 (segment (start 86.733655 129.76) (end 85.81 130.683655) (width 0.8) (layer "B.Cu") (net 7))
 (segment (start 85.81 130.683655) (end 85.81 132.31) (width 0.8) (layer "B.Cu") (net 7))
 (segment (start 99 129.76) (end 86.733655 129.76) (width 0.8) (layer "B.Cu") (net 7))
 (segment (start 61 130.22) (end 61.48628 130.70628) (width 0.8) (layer "F.Cu") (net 4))
 (segment (start 61.48628 130.70628) (end 61.845873 130.70628) (width 0.8) (layer "F.Cu") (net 4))
 (segment (start 63.31464 132) (end 72.8 132) (width 0.8) (layer "F.Cu") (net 4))
 (segment (start 61.845873 130.70628) (end 63.04732 131.907727) (width 0.8) (layer "F.Cu") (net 4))
 (segment (start 72.8 132) (end 73.11 132.31) (width 0.8) (layer "F.Cu") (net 4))
 (segment (start 60.99632 132.75728) (end 61.48532 133.24628) (width 0.8) (layer "F.Cu") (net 5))
 (segment (start 75.225345 134.361) (end 75.65 133.936345) (width 0.8) (layer "F.Cu") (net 5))
 (segment (start 75.65 133.936345) (end 75.65 132.31) (width 0.8) (layer "F.Cu") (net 5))
 (segment (start 62.960593 134.361) (end 75.225345 134.361) (width 0.8) (layer "F.Cu") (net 5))
 (segment (start 61.48532 133.24628) (end 61.845873 133.24628) (width 0.8) (layer "F.Cu") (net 5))
 (segment (start 61.845873 133.24628) (end 62.960593 134.361) (width 0.8) (layer "F.Cu") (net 5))
 (segment (start 88.35 123.063655) (end 88.35 124.69) (width 0.8) (layer "F.Cu") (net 10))
 (segment (start 61 120.06) (end 61.241 120.301) (width 0.8) (layer "F.Cu") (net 10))
 (segment (start 61.241 120.301) (end 85.587345 120.301) (width 0.8) (layer "F.Cu") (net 10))
 (segment (start 85.587345 120.301) (end 88.35 123.063655) (width 0.8) (layer "F.Cu") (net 10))
 (segment (start 90.89 124.69) (end 90.89 123.063655) (width 0.8) (layer "F.Cu") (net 9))
 (segment (start 90.89 123.063655) (end 85.835345 118.009) (width 0.8) (layer "F.Cu") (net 9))
 (segment (start 85.835345 118.009) (end 61.489 118.009) (width 0.8) (layer "F.Cu") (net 9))
 (segment (start 61.489 118.009) (end 61 117.52) (width 0.8) (layer "F.Cu") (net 9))
 (segment (start 75.65 124.15) (end 75.65 124.69) (width 0.8) (layer "F.Cu") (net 13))
 (segment (start 61.978 125.14) (end 64.479 122.639) (width 0.8) (layer "F.Cu") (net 13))
 (segment (start 61 125.14) (end 61.978 125.14) (width 0.8) (layer "F.Cu") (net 13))
 (segment (start 74.139 122.639) (end 75.65 124.15) (width 0.8) (layer "F.Cu") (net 13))
 (segment (start 64.479 122.639) (end 74.139 122.639) (width 0.8) (layer "F.Cu") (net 13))
 (segment (start 88.35 132.670553) (end 88.35 132.31) (width 0.8) (layer "F.Cu") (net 8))
 (segment (start 84.573273 136.44728) (end 88.35 132.670553) (width 0.8) (layer "F.Cu") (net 8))
 (segment (start 62.14632 136.44728) (end 84.573273 136.44728) (width 0.8) (layer "F.Cu") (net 8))
 (segment (start 60.99632 135.29728) (end 62.14632 136.44728) (width 0.8) (layer "F.Cu") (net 8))
 (segment (start 70.15 92.12) (end 61 92.12) (width 0.8) (layer "F.Cu") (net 21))
 (segment (start 76.14 98.11) (end 70.15 92.12) (width 0.8) (layer "F.Cu") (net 21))
 (segment (start 91.482323 100.65) (end 88.84 100.65) (width 0.8) (layer "F.Cu") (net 19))
 (segment (start 98 94.132323) (end 91.482323 100.65) (width 0.8) (layer "F.Cu") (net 19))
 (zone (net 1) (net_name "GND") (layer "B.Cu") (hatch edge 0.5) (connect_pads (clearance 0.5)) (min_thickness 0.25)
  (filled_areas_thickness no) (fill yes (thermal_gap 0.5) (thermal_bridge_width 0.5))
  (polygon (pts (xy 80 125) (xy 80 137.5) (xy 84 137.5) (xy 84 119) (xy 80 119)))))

